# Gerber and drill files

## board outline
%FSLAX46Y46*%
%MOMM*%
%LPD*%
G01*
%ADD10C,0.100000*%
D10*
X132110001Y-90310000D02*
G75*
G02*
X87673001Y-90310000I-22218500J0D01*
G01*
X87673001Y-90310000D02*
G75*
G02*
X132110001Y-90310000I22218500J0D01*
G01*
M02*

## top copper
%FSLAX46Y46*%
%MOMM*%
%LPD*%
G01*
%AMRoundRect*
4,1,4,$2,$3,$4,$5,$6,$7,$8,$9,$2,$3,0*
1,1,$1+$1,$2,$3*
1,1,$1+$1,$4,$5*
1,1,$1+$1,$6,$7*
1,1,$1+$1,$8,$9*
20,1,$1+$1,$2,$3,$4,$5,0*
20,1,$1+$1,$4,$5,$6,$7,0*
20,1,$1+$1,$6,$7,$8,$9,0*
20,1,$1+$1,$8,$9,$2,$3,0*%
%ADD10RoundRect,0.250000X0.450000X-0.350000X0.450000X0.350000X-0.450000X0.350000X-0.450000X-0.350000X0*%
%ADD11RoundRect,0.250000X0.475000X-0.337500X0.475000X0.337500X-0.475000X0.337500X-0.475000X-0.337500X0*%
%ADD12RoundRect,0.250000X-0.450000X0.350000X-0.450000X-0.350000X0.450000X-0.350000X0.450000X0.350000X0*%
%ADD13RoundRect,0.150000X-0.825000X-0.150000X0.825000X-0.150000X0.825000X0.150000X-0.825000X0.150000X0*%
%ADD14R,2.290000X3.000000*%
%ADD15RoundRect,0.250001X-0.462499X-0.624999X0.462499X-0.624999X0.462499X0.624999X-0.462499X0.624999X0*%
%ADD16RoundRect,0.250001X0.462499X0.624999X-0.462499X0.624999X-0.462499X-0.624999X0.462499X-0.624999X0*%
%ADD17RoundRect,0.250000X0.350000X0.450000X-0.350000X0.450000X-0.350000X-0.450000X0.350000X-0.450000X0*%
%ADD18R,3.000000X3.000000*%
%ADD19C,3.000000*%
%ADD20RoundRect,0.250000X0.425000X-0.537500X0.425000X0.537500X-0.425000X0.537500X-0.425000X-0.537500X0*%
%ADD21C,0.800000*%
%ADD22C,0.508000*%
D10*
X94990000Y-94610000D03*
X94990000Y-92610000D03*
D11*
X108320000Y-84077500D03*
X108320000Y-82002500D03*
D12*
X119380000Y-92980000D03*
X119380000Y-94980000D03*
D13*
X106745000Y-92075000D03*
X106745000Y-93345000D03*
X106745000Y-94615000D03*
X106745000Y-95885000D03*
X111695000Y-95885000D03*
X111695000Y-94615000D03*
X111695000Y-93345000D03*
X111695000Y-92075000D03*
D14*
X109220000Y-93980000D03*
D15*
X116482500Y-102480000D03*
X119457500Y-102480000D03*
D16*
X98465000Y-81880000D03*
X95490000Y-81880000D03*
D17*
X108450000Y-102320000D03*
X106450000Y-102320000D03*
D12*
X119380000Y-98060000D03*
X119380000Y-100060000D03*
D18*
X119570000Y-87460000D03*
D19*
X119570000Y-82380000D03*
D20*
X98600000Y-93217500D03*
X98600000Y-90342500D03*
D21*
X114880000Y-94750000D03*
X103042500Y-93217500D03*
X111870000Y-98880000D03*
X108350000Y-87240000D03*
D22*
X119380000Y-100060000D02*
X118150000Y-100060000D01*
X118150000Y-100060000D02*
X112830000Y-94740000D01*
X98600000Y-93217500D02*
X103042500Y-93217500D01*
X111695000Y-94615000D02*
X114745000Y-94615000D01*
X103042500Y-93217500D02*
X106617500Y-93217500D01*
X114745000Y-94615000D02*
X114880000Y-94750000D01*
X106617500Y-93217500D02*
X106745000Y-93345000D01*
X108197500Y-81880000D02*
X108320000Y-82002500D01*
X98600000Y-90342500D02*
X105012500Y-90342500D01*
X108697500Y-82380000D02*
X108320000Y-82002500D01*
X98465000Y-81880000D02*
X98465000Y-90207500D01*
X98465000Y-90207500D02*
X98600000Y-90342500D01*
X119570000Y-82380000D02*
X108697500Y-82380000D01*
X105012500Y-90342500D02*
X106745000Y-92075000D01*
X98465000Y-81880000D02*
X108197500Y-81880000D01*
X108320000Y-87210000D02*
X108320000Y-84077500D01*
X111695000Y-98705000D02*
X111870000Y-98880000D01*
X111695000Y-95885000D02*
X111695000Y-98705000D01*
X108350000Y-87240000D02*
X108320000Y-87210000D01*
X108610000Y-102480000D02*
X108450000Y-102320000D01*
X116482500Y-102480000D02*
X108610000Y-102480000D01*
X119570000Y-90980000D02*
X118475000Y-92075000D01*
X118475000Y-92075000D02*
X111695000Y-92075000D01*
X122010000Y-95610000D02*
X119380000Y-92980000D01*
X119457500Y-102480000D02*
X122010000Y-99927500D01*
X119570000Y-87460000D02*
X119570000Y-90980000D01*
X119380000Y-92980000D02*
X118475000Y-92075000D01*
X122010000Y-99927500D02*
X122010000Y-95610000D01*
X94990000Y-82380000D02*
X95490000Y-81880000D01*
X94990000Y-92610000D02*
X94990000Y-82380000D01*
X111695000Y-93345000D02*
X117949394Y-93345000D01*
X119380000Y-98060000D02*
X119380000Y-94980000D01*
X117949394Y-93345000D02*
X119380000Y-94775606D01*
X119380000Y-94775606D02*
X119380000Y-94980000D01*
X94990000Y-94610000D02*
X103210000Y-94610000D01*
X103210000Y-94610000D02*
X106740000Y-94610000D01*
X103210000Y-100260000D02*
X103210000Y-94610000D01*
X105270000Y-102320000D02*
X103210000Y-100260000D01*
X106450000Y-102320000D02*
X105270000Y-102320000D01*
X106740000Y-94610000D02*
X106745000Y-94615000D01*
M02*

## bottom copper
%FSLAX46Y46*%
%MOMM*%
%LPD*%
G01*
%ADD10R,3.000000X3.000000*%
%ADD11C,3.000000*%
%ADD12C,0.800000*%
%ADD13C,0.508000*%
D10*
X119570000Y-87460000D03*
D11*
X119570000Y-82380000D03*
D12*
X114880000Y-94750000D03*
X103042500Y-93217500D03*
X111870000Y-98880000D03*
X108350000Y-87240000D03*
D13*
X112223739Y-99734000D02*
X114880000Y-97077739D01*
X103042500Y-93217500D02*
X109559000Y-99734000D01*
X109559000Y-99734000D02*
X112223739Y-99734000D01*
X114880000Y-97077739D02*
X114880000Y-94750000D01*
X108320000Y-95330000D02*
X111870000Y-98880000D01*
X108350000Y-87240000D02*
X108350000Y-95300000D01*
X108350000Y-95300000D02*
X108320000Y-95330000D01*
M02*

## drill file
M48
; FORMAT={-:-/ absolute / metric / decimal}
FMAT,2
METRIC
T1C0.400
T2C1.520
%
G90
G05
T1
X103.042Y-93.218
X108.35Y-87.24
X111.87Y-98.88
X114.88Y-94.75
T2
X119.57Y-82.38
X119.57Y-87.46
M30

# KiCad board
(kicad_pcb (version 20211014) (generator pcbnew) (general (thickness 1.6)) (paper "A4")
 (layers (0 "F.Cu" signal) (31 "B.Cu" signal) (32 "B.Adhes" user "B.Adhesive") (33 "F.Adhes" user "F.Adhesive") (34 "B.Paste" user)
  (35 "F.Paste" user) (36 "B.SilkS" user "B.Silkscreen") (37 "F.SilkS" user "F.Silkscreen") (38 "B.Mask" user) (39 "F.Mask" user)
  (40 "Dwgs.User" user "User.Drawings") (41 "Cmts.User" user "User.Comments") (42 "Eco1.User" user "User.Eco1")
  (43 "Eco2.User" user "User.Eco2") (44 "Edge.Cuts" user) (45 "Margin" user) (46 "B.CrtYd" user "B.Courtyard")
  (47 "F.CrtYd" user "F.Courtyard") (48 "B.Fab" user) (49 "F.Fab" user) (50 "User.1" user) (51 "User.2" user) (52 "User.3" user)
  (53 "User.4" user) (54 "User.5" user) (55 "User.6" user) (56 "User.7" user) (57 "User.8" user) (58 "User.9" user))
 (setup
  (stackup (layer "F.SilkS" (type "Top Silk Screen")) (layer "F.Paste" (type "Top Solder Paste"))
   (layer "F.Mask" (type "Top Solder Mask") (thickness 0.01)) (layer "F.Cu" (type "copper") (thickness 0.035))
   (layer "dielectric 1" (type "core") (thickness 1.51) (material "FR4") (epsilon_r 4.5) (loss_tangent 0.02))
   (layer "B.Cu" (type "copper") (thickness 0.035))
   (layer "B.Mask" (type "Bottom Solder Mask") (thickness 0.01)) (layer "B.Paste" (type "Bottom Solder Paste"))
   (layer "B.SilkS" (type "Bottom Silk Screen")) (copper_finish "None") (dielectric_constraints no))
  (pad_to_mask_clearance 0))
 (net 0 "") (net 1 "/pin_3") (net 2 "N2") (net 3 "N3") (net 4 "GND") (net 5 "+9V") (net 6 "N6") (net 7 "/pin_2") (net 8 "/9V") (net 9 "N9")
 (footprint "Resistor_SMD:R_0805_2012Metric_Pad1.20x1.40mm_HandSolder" (layer "F.Cu") (at 94.99 93.61 90)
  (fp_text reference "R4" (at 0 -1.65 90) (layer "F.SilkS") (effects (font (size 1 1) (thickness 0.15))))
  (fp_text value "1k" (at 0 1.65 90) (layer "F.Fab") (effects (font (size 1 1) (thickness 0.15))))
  (pad "1" smd roundrect (at -1 0 90) (size 1.2 1.4) (layers "F.Cu" "F.Paste" "F.Mask") (roundrect_rratio 0.2083333333) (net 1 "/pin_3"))
  (pad "2" smd roundrect (at 1 0 90) (size 1.2 1.4) (layers "F.Cu" "F.Paste" "F.Mask") (roundrect_rratio 0.2083333333) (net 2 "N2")))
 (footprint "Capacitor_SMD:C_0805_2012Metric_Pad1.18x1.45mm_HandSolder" (layer "F.Cu") (at 108.32 83.04 90)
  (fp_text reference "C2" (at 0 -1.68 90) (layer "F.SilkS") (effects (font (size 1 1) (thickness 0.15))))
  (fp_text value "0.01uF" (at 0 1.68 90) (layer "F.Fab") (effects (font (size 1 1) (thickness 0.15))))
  (pad "1" smd roundrect (at -1.0375 0 90) (size 1.175 1.45) (layers "F.Cu" "F.Paste" "F.Mask") (roundrect_rratio 0.2127659574) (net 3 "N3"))
  (pad "2" smd roundrect (at 1.0375 0 90) (size 1.175 1.45) (layers "F.Cu" "F.Paste" "F.Mask") (roundrect_rratio 0.2127659574) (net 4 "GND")))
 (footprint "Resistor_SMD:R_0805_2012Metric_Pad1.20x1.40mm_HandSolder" (layer "F.Cu") (at 119.38 93.98 -90)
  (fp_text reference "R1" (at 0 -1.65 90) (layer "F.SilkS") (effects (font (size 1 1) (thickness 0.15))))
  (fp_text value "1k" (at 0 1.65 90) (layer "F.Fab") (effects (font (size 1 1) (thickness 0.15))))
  (pad "1" smd roundrect (at -1 0 270) (size 1.2 1.4) (layers "F.Cu" "F.Paste" "F.Mask") (roundrect_rratio 0.2083333333) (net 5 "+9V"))
  (pad "2" smd roundrect (at 1 0 270) (size 1.2 1.4) (layers "F.Cu" "F.Paste" "F.Mask") (roundrect_rratio 0.2083333333) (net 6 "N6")))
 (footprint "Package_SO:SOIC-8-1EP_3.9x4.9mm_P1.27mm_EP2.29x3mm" (layer "F.Cu") (at 109.22 93.98)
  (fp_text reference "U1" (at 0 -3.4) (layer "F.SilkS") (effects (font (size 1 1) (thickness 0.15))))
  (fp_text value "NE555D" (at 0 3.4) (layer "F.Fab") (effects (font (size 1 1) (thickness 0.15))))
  (pad "" smd roundrect (at -0.57 -0.75) (size 0.92 1.21) (layers "F.Paste") (roundrect_rratio 0.25))
  (pad "" smd roundrect (at -0.57 0.75) (size 0.92 1.21) (layers "F.Paste") (roundrect_rratio 0.25))
  (pad "" smd roundrect (at 0.57 0.75) (size 0.92 1.21) (layers "F.Paste") (roundrect_rratio 0.25))
  (pad "" smd roundrect (at 0.57 -0.75) (size 0.92 1.21) (layers "F.Paste") (roundrect_rratio 0.25))
  (pad "1" smd roundrect (at -2.475 -1.905) (size 1.95 0.6) (layers "F.Cu" "F.Paste" "F.Mask") (roundrect_rratio 0.25) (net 4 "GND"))
  (pad "2" smd roundrect (at -2.475 -0.635) (size 1.95 0.6) (layers "F.Cu" "F.Paste" "F.Mask") (roundrect_rratio 0.25) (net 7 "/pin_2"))
  (pad "3" smd roundrect (at -2.475 0.635) (size 1.95 0.6) (layers "F.Cu" "F.Paste" "F.Mask") (roundrect_rratio 0.25) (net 1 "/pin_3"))
  (pad "4" smd roundrect (at -2.475 1.905) (size 1.95 0.6) (layers "F.Cu" "F.Paste" "F.Mask") (roundrect_rratio 0.25) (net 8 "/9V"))
  (pad "5" smd roundrect (at 2.475 1.905) (size 1.95 0.6) (layers "F.Cu" "F.Paste" "F.Mask") (roundrect_rratio 0.25) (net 3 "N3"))
  (pad "6" smd roundrect (at 2.475 0.635) (size 1.95 0.6) (layers "F.Cu" "F.Paste" "F.Mask") (roundrect_rratio 0.25) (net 7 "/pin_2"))
  (pad "7" smd roundrect (at 2.475 -0.635) (size 1.95 0.6) (layers "F.Cu" "F.Paste" "F.Mask") (roundrect_rratio 0.25) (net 6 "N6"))
  (pad "8" smd roundrect (at 2.475 -1.905) (size 1.95 0.6) (layers "F.Cu" "F.Paste" "F.Mask") (roundrect_rratio 0.25) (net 5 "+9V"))
  (pad "9" smd rect (at 0 0) (size 2.29 3) (layers "F.Cu" "F.Mask")))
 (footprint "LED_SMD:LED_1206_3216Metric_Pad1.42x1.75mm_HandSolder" (layer "F.Cu") (at 117.97 102.48)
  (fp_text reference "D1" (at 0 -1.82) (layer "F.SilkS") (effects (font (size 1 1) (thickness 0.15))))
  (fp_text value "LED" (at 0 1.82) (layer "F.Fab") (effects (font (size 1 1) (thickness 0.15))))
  (pad "1" smd roundrect (at -1.4875 0) (size 1.425 1.75) (layers "F.Cu" "F.Paste" "F.Mask") (roundrect_rratio 0.1754392982) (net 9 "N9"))
  (pad "2" smd roundrect (at 1.4875 0) (size 1.425 1.75) (layers "F.Cu" "F.Paste" "F.Mask") (roundrect_rratio 0.1754392982) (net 5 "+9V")))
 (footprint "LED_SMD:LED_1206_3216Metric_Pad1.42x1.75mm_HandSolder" (layer "F.Cu") (at 96.9775 81.88 180)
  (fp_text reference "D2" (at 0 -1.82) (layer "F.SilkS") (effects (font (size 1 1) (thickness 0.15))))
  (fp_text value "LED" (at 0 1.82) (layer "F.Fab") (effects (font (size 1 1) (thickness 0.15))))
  (pad "1" smd roundrect (at -1.4875 0 180) (size 1.425 1.75) (layers "F.Cu" "F.Paste" "F.Mask") (roundrect_rratio 0.1754392982)
   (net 4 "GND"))
  (pad "2" smd roundrect (at 1.4875 0 180) (size 1.425 1.75) (layers "F.Cu" "F.Paste" "F.Mask") (roundrect_rratio 0.1754392982) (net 2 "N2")))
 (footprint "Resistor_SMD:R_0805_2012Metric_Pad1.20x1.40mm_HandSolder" (layer "F.Cu") (at 107.45 102.32 180)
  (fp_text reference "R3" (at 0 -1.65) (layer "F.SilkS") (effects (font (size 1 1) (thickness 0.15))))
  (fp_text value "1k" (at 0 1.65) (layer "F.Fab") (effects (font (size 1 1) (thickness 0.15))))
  (pad "1" smd roundrect (at -1 0 180) (size 1.2 1.4) (layers "F.Cu" "F.Paste" "F.Mask") (roundrect_rratio 0.2083333333) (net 9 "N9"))
  (pad "2" smd roundrect (at 1 0 180) (size 1.2 1.4) (layers "F.Cu" "F.Paste" "F.Mask") (roundrect_rratio 0.2083333333) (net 1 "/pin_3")))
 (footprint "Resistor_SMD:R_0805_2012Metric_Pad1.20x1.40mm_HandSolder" (layer "F.Cu") (at 119.38 99.06 -90)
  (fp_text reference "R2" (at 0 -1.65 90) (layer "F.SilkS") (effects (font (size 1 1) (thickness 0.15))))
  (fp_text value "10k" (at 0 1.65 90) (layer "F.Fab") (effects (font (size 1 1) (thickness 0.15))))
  (pad "1" smd roundrect (at -1 0 270) (size 1.2 1.4) (layers "F.Cu" "F.Paste" "F.Mask") (roundrect_rratio 0.2083333333) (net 6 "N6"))
  (pad "2" smd roundrect (at 1 0 270) (size 1.2 1.4) (layers "F.Cu" "F.Paste" "F.Mask") (roundrect_rratio 0.2083333333) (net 7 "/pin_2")))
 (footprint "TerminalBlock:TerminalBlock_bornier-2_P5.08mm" (layer "F.Cu") (at 119.57 87.46 90)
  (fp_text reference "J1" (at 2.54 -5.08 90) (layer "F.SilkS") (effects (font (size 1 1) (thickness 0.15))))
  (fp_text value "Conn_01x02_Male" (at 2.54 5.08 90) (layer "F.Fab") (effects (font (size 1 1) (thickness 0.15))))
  (pad "1" thru_hole rect (at 0 0 90) (size 3 3) (drill 1.52) (layers *.Cu *.Mask) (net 5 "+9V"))
  (pad "2" thru_hole circle (at 5.08 0 90) (size 3 3) (drill 1.52) (layers *.Cu *.Mask) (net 4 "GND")))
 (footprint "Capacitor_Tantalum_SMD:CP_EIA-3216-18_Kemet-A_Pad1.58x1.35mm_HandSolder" (layer "F.Cu") (at 98.6 91.78 90)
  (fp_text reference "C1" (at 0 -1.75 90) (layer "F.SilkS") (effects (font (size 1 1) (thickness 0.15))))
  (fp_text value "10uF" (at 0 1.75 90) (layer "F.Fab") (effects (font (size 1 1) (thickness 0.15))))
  (pad "1" smd roundrect (at -1.4375 0 90) (size 1.575 1.35) (layers "F.Cu" "F.Paste" "F.Mask") (roundrect_rratio 0.1851851852)
   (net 7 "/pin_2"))
  (pad "2" smd roundrect (at 1.4375 0 90) (size 1.575 1.35) (layers "F.Cu" "F.Paste" "F.Mask") (roundrect_rratio 0.1851851852) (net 4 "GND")))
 (gr_circle (center 109.891501 90.31) (end 129.890484 80.63) (layer "Edge.Cuts") (width 0.1) (fill none))
 (segment (start 119.38 100.06) (end 118.15 100.06) (width 0.508) (layer "F.Cu") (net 7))
 (segment (start 118.15 100.06) (end 112.83 94.74) (width 0.508) (layer "F.Cu") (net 7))
 (segment (start 98.6 93.2175) (end 103.0425 93.2175) (width 0.508) (layer "F.Cu") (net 7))
 (segment (start 111.695 94.615) (end 114.745 94.615) (width 0.508) (layer "F.Cu") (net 7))
 (segment (start 103.0425 93.2175) (end 106.6175 93.2175) (width 0.508) (layer "F.Cu") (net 7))
 (segment (start 114.745 94.615) (end 114.88 94.75) (width 0.508) (layer "F.Cu") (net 7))
 (segment (start 106.6175 93.2175) (end 106.745 93.345) (width 0.508) (layer "F.Cu") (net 7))
 (via (at 114.88 94.75) (size 0.8) (drill 0.4) (layers "F.Cu" "B.Cu") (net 7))
 (via (at 103.0425 93.2175) (size 0.8) (drill 0.4) (layers "F.Cu" "B.Cu") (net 7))
 (segment (start 112.223739 99.734) (end 114.88 97.077739) (width 0.508) (layer "B.Cu") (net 7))
 (segment (start 103.0425 93.2175) (end 109.559 99.734) (width 0.508) (layer "B.Cu") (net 7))
 (segment (start 109.559 99.734) (end 112.223739 99.734) (width 0.508) (layer "B.Cu") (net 7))
 (segment (start 114.88 97.077739) (end 114.88 94.75) (width 0.508) (layer "B.Cu") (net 7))
 (segment (start 108.1975 81.88) (end 108.32 82.0025) (width 0.508) (layer "F.Cu") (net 4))
 (segment (start 98.6 90.3425) (end 105.0125 90.3425) (width 0.508) (layer "F.Cu") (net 4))
 (segment (start 108.6975 82.38) (end 108.32 82.0025) (width 0.508) (layer "F.Cu") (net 4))
 (segment (start 98.465 81.88) (end 98.465 90.2075) (width 0.508) (layer "F.Cu") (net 4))
 (segment (start 98.465 90.2075) (end 98.6 90.3425) (width 0.508) (layer "F.Cu") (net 4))
 (segment (start 119.57 82.38) (end 108.6975 82.38) (width 0.508) (layer "F.Cu") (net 4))
 (segment (start 105.0125 90.3425) (end 106.745 92.075) (width 0.508) (layer "F.Cu") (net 4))
 (segment (start 98.465 81.88) (end 108.1975 81.88) (width 0.508) (layer "F.Cu") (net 4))
 (segment (start 108.32 87.21) (end 108.32 84.0775) (width 0.508) (layer "F.Cu") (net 3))
 (segment (start 111.695 98.705) (end 111.87 98.88) (width 0.508) (layer "F.Cu") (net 3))
 (segment (start 111.695 95.885) (end 111.695 98.705) (width 0.508) (layer "F.Cu") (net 3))
 (segment (start 108.35 87.24) (end 108.32 87.21) (width 0.508) (layer "F.Cu") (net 3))
 (via (at 111.87 98.88) (size 0.8) (drill 0.4) (layers "F.Cu" "B.Cu") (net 3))
 (via (at 108.35 87.24) (size 0.8) (drill 0.4) (layers "F.Cu" "B.Cu") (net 3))
 (segment (start 108.32 95.33) (end 111.87 98.88) (width 0.508) (layer "B.Cu") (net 3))
 (segment (start 108.35 87.24) (end 108.35 95.3) (width 0.508) (layer "B.Cu") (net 3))
 (segment (start 108.35 95.3) (end 108.32 95.33) (width 0.508) (layer "B.Cu") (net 3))
 (segment (start 108.61 102.48) (end 108.45 102.32) (width 0.508) (layer "F.Cu") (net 9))
 (segment (start 116.4825 102.48) (end 108.61 102.48) (width 0.508) (layer "F.Cu") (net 9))
 (segment (start 119.57 90.98) (end 118.475 92.075) (width 0.508) (layer "F.Cu") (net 5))
 (segment (start 118.475 92.075) (end 111.695 92.075) (width 0.508) (layer "F.Cu") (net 5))
 (segment (start 122.01 95.61) (end 119.38 92.98) (width 0.508) (layer "F.Cu") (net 5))
 (segment (start 119.4575 102.48) (end 122.01 99.9275) (width 0.508) (layer "F.Cu") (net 5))
 (segment (start 119.57 87.46) (end 119.57 90.98) (width 0.508) (layer "F.Cu") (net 5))
 (segment (start 119.38 92.98) (end 118.475 92.075) (width 0.508) (layer "F.Cu") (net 5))
 (segment (start 122.01 99.9275) (end 122.01 95.61) (width 0.508) (layer "F.Cu") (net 5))
 (segment (start 94.99 82.38) (end 95.49 81.88) (width 0.508) (layer "F.Cu") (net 2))
 (segment (start 94.99 92.61) (end 94.99 82.38) (width 0.508) (layer "F.Cu") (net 2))
 (segment (start 111.695 93.345) (end 117.949394 93.345) (width 0.508) (layer "F.Cu") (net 6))
 (segment (start 119.38 98.06) (end 119.38 94.98) (width 0.508) (layer "F.Cu") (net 6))
 (segment (start 117.949394 93.345) (end 119.38 94.775606) (width 0.508) (layer "F.Cu") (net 6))
 (segment (start 119.38 94.775606) (end 119.38 94.98) (width 0.508) (layer "F.Cu") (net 6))
 (segment (start 94.99 94.61) (end 103.21 94.61) (width 0.508) (layer "F.Cu") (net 1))
 (segment (start 103.21 94.61) (end 106.74 94.61) (width 0.508) (layer "F.Cu") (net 1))
 (segment (start 103.21 100.26) (end 103.21 94.61) (width 0.508) (layer "F.Cu") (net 1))
 (segment (start 105.27 102.32) (end 103.21 100.26) (width 0.508) (layer "F.Cu") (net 1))
 (segment (start 106.45 102.32) (end 105.27 102.32) (width 0.508) (layer "F.Cu") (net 1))
 (segment (start 106.74 94.61) (end 106.745 94.615) (width 0.508) (layer "F.Cu") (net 1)))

